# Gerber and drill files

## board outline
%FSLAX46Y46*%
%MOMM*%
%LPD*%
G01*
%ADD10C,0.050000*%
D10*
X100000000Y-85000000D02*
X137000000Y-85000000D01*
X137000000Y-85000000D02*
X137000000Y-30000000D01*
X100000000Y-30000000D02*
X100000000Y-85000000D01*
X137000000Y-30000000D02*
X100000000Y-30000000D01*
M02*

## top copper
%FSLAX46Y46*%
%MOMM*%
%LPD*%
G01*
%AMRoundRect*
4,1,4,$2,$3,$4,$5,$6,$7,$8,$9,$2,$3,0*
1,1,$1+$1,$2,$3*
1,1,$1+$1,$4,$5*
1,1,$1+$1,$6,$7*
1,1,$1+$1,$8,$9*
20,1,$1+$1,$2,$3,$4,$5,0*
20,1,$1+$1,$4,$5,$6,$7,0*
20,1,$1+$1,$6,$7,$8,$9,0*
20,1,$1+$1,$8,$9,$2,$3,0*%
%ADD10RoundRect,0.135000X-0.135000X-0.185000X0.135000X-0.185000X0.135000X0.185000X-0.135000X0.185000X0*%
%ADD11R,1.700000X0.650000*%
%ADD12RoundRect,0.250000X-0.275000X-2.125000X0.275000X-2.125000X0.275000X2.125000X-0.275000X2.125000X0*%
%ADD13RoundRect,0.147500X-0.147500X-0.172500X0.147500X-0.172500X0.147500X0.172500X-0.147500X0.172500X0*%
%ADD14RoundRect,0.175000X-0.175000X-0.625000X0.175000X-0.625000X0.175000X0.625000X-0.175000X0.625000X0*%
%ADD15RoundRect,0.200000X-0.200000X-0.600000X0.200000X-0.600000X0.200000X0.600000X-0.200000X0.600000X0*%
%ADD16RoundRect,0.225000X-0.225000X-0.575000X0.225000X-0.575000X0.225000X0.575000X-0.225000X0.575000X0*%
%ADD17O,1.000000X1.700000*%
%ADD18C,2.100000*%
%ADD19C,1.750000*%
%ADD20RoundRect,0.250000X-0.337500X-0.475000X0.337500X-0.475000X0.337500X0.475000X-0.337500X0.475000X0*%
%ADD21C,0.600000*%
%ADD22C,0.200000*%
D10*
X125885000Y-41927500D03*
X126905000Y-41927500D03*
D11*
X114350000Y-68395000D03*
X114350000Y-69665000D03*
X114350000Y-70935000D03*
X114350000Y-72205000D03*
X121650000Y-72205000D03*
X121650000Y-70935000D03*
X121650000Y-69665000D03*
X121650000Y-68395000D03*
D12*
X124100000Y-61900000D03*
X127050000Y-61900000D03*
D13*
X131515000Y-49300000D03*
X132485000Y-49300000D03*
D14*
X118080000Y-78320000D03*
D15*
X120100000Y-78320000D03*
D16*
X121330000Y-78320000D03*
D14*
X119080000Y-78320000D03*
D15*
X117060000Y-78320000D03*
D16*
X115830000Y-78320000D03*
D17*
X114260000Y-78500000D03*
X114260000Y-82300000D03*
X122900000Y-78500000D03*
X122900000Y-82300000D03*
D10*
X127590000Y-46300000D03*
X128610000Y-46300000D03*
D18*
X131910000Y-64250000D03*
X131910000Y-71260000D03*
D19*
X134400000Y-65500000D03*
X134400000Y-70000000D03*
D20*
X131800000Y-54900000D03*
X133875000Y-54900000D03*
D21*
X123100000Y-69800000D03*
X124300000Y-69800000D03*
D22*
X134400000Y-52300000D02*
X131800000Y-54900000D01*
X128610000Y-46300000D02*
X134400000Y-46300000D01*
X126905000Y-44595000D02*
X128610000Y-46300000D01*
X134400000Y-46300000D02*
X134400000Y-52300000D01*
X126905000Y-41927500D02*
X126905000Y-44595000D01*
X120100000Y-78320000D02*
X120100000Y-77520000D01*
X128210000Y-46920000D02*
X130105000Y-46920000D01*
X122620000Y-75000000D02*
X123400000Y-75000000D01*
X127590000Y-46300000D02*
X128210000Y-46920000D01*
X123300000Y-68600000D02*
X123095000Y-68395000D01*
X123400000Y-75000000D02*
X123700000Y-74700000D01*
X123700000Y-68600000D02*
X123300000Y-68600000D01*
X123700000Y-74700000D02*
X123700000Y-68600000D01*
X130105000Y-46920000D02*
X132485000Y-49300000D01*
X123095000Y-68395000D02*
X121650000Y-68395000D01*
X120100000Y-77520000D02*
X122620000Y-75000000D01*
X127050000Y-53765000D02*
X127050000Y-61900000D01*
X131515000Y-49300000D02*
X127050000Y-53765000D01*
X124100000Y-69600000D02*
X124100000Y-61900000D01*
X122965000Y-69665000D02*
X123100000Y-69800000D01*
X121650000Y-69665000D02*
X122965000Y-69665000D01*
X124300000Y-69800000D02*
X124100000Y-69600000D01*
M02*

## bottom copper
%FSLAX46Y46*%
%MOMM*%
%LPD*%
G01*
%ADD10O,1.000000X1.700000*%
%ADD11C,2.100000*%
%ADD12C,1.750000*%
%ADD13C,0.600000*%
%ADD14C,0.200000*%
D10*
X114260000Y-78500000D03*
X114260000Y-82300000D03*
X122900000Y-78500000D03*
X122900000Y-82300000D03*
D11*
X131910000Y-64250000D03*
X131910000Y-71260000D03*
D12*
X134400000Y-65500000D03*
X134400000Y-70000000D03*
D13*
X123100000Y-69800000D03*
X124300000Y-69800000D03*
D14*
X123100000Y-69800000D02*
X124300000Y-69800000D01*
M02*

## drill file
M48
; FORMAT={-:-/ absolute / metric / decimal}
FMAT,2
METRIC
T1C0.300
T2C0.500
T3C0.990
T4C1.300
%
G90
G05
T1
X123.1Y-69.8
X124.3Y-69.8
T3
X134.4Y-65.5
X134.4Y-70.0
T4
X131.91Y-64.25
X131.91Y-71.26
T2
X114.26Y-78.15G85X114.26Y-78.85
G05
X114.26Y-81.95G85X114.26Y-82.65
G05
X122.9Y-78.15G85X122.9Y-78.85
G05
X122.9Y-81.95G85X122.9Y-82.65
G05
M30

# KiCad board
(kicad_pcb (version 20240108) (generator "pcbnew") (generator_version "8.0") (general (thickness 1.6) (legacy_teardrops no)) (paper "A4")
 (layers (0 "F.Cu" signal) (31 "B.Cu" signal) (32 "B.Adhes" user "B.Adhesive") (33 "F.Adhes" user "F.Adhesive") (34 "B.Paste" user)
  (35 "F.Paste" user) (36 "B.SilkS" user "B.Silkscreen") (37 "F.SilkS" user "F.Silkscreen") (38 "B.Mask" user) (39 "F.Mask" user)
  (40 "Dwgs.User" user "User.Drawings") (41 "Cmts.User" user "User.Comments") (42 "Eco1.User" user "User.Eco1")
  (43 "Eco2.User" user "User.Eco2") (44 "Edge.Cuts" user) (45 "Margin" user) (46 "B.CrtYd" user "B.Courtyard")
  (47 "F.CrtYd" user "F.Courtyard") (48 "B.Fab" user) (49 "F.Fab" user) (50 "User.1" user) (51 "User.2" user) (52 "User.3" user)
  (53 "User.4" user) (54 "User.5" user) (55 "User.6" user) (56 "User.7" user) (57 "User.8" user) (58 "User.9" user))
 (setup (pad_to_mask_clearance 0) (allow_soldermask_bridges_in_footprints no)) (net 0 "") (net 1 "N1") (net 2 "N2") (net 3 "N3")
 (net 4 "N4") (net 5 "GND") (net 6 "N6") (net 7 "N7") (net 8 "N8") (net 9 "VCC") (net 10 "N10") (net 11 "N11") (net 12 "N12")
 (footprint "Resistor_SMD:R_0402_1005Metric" (layer "F.Cu") (at 126.395 41.9275)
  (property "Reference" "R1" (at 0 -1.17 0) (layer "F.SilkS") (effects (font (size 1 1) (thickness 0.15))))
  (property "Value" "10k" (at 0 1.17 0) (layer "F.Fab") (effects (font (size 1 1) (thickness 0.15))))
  (pad "1" smd roundrect (at -0.51 0) (size 0.54 0.64) (layers "F.Cu" "F.Paste" "F.Mask") (roundrect_rratio 0.25) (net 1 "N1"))
  (pad "2" smd roundrect (at 0.51 0) (size 0.54 0.64) (layers "F.Cu" "F.Paste" "F.Mask") (roundrect_rratio 0.25) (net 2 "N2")))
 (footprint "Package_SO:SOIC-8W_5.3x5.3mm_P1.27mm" (layer "F.Cu") (at 118 70.3)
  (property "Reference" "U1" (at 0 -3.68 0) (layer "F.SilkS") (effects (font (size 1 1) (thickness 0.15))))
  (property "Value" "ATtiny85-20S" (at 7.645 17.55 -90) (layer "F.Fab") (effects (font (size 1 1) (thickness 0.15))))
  (pad "1" smd rect (at -3.65 -1.905) (size 1.7 0.65) (layers "F.Cu" "F.Paste" "F.Mask") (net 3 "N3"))
  (pad "2" smd rect (at -3.65 -0.635) (size 1.7 0.65) (layers "F.Cu" "F.Paste" "F.Mask") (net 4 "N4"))
  (pad "3" smd rect (at -3.65 0.635) (size 1.7 0.65) (layers "F.Cu" "F.Paste" "F.Mask") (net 1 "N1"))
  (pad "4" smd rect (at -3.65 1.905) (size 1.7 0.65) (layers "F.Cu" "F.Paste" "F.Mask") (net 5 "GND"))
  (pad "5" smd rect (at 3.65 1.905) (size 1.7 0.65) (layers "F.Cu" "F.Paste" "F.Mask") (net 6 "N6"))
  (pad "6" smd rect (at 3.65 0.635) (size 1.7 0.65) (layers "F.Cu" "F.Paste" "F.Mask") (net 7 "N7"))
  (pad "7" smd rect (at 3.65 -0.635) (size 1.7 0.65) (layers "F.Cu" "F.Paste" "F.Mask") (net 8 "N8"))
  (pad "8" smd rect (at 3.65 -1.905) (size 1.7 0.65) (layers "F.Cu" "F.Paste" "F.Mask") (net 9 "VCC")))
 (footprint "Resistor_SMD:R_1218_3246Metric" (layer "F.Cu") (at 125.575 61.9)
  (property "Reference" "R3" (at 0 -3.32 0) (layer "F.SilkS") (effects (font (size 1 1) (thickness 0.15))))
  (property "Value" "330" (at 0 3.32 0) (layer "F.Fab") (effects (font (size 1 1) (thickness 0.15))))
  (pad "1" smd roundrect (at -1.475 0) (size 1.05 4.75) (layers "F.Cu" "F.Paste" "F.Mask") (roundrect_rratio 0.238095) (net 8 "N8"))
  (pad "2" smd roundrect (at 1.475 0) (size 1.05 4.75) (layers "F.Cu" "F.Paste" "F.Mask") (roundrect_rratio 0.238095) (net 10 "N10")))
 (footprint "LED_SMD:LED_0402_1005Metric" (layer "F.Cu") (at 132 49.3)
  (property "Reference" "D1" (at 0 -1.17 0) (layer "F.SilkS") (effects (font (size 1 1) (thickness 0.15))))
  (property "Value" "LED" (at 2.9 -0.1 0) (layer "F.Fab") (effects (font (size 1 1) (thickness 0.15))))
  (pad "1" smd roundrect (at -0.485 0) (size 0.59 0.64) (layers "F.Cu" "F.Paste" "F.Mask") (roundrect_rratio 0.25) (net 10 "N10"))
  (pad "2" smd roundrect (at 0.485 0) (size 0.59 0.64) (layers "F.Cu" "F.Paste" "F.Mask") (roundrect_rratio 0.25) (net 9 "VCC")))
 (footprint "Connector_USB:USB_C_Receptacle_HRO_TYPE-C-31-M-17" (layer "F.Cu") (at 118.58 81.5)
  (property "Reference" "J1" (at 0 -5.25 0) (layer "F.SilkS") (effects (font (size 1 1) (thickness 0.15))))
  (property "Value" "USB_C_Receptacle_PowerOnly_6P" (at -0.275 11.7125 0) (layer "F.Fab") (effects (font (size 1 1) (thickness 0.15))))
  (pad "A5" smd roundrect (at -0.5 -3.18) (size 0.7 1.6) (layers "F.Cu" "F.Paste" "F.Mask") (roundrect_rratio 0.25) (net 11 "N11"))
  (pad "A9" smd roundrect (at 1.52 -3.18) (size 0.8 1.6) (layers "F.Cu" "F.Paste" "F.Mask") (roundrect_rratio 0.25) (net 9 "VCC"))
  (pad "A12" smd roundrect (at 2.75 -3.18) (size 0.9 1.6) (layers "F.Cu" "F.Paste" "F.Mask") (roundrect_rratio 0.25) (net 5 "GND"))
  (pad "B5" smd roundrect (at 0.5 -3.18) (size 0.7 1.6) (layers "F.Cu" "F.Paste" "F.Mask") (roundrect_rratio 0.25) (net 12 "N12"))
  (pad "B9" smd roundrect (at -1.52 -3.18) (size 0.8 1.6) (layers "F.Cu" "F.Paste" "F.Mask") (roundrect_rratio 0.25) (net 9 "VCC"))
  (pad "B12" smd roundrect (at -2.75 -3.18) (size 0.9 1.6) (layers "F.Cu" "F.Paste" "F.Mask") (roundrect_rratio 0.25) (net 5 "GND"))
  (pad "S1" thru_hole oval (at -4.32 -3) (size 1 1.7) (drill oval 0.5 1.2) (layers "*.Cu" "*.Mask") (remove_unused_layers no) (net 5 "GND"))
  (pad "S1" thru_hole oval (at -4.32 0.8) (size 1 1.7) (drill oval 0.5 1.2) (layers "*.Cu" "*.Mask") (remove_unused_layers no) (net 5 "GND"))
  (pad "S1" thru_hole oval (at 4.32 -3) (size 1 1.7) (drill oval 0.5 1.2) (layers "*.Cu" "*.Mask") (remove_unused_layers no) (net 5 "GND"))
  (pad "S1" thru_hole oval (at 4.32 0.8) (size 1 1.7) (drill oval 0.5 1.2) (layers "*.Cu" "*.Mask") (remove_unused_layers no) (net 5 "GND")))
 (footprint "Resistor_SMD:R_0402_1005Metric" (layer "F.Cu") (at 128.1 46.3)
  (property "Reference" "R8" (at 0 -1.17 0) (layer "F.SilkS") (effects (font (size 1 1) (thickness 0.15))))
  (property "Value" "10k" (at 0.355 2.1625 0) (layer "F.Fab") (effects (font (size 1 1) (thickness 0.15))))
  (pad "1" smd roundrect (at -0.51 0) (size 0.54 0.64) (layers "F.Cu" "F.Paste" "F.Mask") (roundrect_rratio 0.25) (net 9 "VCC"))
  (pad "2" smd roundrect (at 0.51 0) (size 0.54 0.64) (layers "F.Cu" "F.Paste" "F.Mask") (roundrect_rratio 0.25) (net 2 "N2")))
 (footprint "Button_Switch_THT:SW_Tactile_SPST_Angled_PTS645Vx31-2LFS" (layer "F.Cu") (at 134.4 65.5 -90)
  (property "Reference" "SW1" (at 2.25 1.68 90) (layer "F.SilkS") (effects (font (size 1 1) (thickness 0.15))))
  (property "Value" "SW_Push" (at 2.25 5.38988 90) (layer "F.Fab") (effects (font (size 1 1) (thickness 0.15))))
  (pad "" thru_hole circle (at -1.25 2.49 270) (size 2.1 2.1) (drill 1.3) (layers "*.Cu" "*.Mask") (remove_unused_layers no))
  (pad "" thru_hole circle (at 5.76 2.49 270) (size 2.1 2.1) (drill 1.3) (layers "*.Cu" "*.Mask") (remove_unused_layers no))
  (pad "1" thru_hole circle (at 0 0 270) (size 1.75 1.75) (drill 0.99) (layers "*.Cu" "*.Mask") (remove_unused_layers no) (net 5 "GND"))
  (pad "2" thru_hole circle (at 4.5 0 270) (size 1.75 1.75) (drill 0.99) (layers "*.Cu" "*.Mask") (remove_unused_layers no) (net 2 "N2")))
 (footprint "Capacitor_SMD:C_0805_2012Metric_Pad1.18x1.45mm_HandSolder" (layer "F.Cu") (at 132.8375 54.9)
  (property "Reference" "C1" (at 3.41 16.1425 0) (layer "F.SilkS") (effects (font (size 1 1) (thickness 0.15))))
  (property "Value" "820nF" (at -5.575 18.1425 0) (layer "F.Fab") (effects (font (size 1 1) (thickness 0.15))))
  (pad "1" smd roundrect (at -1.0375 0) (size 1.175 1.45) (layers "F.Cu" "F.Paste" "F.Mask") (roundrect_rratio 0.212766) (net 2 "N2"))
  (pad "2" smd roundrect (at 1.0375 0) (size 1.175 1.45) (layers "F.Cu" "F.Paste" "F.Mask") (roundrect_rratio 0.212766) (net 5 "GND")))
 (gr_line (start 100 85) (end 137 85) (stroke (width 0.05) (type default)) (layer "Edge.Cuts"))
 (gr_line (start 137 85) (end 137 30) (stroke (width 0.05) (type default)) (layer "Edge.Cuts"))
 (gr_line (start 100 30) (end 100 85) (stroke (width 0.05) (type default)) (layer "Edge.Cuts"))
 (gr_line (start 137 30) (end 100 30) (stroke (width 0.05) (type default)) (layer "Edge.Cuts"))
 (segment (start 134.4 52.3) (end 131.8 54.9) (width 0.2) (layer "F.Cu") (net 2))
 (segment (start 128.61 46.3) (end 134.4 46.3) (width 0.2) (layer "F.Cu") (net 2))
 (segment (start 126.905 44.595) (end 128.61 46.3) (width 0.2) (layer "F.Cu") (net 2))
 (segment (start 134.4 46.3) (end 134.4 52.3) (width 0.2) (layer "F.Cu") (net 2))
 (segment (start 126.905 41.9275) (end 126.905 44.595) (width 0.2) (layer "F.Cu") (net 2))
 (segment (start 120.1 78.32) (end 120.1 77.52) (width 0.2) (layer "F.Cu") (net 9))
 (segment (start 128.21 46.92) (end 130.105 46.92) (width 0.2) (layer "F.Cu") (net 9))
 (segment (start 122.62 75) (end 123.4 75) (width 0.2) (layer "F.Cu") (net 9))
 (segment (start 127.59 46.3) (end 128.21 46.92) (width 0.2) (layer "F.Cu") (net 9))
 (segment (start 123.3 68.6) (end 123.095 68.395) (width 0.2) (layer "F.Cu") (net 9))
 (segment (start 123.4 75) (end 123.7 74.7) (width 0.2) (layer "F.Cu") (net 9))
 (segment (start 123.7 68.6) (end 123.3 68.6) (width 0.2) (layer "F.Cu") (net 9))
 (segment (start 123.7 74.7) (end 123.7 68.6) (width 0.2) (layer "F.Cu") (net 9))
 (segment (start 130.105 46.92) (end 132.485 49.3) (width 0.2) (layer "F.Cu") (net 9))
 (segment (start 123.095 68.395) (end 121.65 68.395) (width 0.2) (layer "F.Cu") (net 9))
 (segment (start 120.1 77.52) (end 122.62 75) (width 0.2) (layer "F.Cu") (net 9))
 (segment (start 127.05 53.765) (end 127.05 61.9) (width 0.2) (layer "F.Cu") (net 10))
 (segment (start 131.515 49.3) (end 127.05 53.765) (width 0.2) (layer "F.Cu") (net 10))
 (segment (start 124.1 69.6) (end 124.1 61.9) (width 0.2) (layer "F.Cu") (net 8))
 (segment (start 122.965 69.665) (end 123.1 69.8) (width 0.2) (layer "F.Cu") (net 8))
 (segment (start 121.65 69.665) (end 122.965 69.665) (width 0.2) (layer "F.Cu") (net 8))
 (segment (start 124.3 69.8) (end 124.1 69.6) (width 0.2) (layer "F.Cu") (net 8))
 (via (at 123.1 69.8) (size 0.6) (drill 0.3) (layers "F.Cu" "B.Cu") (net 8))
 (via (at 124.3 69.8) (size 0.6) (drill 0.3) (layers "F.Cu" "B.Cu") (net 8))
 (segment (start 123.1 69.8) (end 124.3 69.8) (width 0.2) (layer "B.Cu") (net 8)))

